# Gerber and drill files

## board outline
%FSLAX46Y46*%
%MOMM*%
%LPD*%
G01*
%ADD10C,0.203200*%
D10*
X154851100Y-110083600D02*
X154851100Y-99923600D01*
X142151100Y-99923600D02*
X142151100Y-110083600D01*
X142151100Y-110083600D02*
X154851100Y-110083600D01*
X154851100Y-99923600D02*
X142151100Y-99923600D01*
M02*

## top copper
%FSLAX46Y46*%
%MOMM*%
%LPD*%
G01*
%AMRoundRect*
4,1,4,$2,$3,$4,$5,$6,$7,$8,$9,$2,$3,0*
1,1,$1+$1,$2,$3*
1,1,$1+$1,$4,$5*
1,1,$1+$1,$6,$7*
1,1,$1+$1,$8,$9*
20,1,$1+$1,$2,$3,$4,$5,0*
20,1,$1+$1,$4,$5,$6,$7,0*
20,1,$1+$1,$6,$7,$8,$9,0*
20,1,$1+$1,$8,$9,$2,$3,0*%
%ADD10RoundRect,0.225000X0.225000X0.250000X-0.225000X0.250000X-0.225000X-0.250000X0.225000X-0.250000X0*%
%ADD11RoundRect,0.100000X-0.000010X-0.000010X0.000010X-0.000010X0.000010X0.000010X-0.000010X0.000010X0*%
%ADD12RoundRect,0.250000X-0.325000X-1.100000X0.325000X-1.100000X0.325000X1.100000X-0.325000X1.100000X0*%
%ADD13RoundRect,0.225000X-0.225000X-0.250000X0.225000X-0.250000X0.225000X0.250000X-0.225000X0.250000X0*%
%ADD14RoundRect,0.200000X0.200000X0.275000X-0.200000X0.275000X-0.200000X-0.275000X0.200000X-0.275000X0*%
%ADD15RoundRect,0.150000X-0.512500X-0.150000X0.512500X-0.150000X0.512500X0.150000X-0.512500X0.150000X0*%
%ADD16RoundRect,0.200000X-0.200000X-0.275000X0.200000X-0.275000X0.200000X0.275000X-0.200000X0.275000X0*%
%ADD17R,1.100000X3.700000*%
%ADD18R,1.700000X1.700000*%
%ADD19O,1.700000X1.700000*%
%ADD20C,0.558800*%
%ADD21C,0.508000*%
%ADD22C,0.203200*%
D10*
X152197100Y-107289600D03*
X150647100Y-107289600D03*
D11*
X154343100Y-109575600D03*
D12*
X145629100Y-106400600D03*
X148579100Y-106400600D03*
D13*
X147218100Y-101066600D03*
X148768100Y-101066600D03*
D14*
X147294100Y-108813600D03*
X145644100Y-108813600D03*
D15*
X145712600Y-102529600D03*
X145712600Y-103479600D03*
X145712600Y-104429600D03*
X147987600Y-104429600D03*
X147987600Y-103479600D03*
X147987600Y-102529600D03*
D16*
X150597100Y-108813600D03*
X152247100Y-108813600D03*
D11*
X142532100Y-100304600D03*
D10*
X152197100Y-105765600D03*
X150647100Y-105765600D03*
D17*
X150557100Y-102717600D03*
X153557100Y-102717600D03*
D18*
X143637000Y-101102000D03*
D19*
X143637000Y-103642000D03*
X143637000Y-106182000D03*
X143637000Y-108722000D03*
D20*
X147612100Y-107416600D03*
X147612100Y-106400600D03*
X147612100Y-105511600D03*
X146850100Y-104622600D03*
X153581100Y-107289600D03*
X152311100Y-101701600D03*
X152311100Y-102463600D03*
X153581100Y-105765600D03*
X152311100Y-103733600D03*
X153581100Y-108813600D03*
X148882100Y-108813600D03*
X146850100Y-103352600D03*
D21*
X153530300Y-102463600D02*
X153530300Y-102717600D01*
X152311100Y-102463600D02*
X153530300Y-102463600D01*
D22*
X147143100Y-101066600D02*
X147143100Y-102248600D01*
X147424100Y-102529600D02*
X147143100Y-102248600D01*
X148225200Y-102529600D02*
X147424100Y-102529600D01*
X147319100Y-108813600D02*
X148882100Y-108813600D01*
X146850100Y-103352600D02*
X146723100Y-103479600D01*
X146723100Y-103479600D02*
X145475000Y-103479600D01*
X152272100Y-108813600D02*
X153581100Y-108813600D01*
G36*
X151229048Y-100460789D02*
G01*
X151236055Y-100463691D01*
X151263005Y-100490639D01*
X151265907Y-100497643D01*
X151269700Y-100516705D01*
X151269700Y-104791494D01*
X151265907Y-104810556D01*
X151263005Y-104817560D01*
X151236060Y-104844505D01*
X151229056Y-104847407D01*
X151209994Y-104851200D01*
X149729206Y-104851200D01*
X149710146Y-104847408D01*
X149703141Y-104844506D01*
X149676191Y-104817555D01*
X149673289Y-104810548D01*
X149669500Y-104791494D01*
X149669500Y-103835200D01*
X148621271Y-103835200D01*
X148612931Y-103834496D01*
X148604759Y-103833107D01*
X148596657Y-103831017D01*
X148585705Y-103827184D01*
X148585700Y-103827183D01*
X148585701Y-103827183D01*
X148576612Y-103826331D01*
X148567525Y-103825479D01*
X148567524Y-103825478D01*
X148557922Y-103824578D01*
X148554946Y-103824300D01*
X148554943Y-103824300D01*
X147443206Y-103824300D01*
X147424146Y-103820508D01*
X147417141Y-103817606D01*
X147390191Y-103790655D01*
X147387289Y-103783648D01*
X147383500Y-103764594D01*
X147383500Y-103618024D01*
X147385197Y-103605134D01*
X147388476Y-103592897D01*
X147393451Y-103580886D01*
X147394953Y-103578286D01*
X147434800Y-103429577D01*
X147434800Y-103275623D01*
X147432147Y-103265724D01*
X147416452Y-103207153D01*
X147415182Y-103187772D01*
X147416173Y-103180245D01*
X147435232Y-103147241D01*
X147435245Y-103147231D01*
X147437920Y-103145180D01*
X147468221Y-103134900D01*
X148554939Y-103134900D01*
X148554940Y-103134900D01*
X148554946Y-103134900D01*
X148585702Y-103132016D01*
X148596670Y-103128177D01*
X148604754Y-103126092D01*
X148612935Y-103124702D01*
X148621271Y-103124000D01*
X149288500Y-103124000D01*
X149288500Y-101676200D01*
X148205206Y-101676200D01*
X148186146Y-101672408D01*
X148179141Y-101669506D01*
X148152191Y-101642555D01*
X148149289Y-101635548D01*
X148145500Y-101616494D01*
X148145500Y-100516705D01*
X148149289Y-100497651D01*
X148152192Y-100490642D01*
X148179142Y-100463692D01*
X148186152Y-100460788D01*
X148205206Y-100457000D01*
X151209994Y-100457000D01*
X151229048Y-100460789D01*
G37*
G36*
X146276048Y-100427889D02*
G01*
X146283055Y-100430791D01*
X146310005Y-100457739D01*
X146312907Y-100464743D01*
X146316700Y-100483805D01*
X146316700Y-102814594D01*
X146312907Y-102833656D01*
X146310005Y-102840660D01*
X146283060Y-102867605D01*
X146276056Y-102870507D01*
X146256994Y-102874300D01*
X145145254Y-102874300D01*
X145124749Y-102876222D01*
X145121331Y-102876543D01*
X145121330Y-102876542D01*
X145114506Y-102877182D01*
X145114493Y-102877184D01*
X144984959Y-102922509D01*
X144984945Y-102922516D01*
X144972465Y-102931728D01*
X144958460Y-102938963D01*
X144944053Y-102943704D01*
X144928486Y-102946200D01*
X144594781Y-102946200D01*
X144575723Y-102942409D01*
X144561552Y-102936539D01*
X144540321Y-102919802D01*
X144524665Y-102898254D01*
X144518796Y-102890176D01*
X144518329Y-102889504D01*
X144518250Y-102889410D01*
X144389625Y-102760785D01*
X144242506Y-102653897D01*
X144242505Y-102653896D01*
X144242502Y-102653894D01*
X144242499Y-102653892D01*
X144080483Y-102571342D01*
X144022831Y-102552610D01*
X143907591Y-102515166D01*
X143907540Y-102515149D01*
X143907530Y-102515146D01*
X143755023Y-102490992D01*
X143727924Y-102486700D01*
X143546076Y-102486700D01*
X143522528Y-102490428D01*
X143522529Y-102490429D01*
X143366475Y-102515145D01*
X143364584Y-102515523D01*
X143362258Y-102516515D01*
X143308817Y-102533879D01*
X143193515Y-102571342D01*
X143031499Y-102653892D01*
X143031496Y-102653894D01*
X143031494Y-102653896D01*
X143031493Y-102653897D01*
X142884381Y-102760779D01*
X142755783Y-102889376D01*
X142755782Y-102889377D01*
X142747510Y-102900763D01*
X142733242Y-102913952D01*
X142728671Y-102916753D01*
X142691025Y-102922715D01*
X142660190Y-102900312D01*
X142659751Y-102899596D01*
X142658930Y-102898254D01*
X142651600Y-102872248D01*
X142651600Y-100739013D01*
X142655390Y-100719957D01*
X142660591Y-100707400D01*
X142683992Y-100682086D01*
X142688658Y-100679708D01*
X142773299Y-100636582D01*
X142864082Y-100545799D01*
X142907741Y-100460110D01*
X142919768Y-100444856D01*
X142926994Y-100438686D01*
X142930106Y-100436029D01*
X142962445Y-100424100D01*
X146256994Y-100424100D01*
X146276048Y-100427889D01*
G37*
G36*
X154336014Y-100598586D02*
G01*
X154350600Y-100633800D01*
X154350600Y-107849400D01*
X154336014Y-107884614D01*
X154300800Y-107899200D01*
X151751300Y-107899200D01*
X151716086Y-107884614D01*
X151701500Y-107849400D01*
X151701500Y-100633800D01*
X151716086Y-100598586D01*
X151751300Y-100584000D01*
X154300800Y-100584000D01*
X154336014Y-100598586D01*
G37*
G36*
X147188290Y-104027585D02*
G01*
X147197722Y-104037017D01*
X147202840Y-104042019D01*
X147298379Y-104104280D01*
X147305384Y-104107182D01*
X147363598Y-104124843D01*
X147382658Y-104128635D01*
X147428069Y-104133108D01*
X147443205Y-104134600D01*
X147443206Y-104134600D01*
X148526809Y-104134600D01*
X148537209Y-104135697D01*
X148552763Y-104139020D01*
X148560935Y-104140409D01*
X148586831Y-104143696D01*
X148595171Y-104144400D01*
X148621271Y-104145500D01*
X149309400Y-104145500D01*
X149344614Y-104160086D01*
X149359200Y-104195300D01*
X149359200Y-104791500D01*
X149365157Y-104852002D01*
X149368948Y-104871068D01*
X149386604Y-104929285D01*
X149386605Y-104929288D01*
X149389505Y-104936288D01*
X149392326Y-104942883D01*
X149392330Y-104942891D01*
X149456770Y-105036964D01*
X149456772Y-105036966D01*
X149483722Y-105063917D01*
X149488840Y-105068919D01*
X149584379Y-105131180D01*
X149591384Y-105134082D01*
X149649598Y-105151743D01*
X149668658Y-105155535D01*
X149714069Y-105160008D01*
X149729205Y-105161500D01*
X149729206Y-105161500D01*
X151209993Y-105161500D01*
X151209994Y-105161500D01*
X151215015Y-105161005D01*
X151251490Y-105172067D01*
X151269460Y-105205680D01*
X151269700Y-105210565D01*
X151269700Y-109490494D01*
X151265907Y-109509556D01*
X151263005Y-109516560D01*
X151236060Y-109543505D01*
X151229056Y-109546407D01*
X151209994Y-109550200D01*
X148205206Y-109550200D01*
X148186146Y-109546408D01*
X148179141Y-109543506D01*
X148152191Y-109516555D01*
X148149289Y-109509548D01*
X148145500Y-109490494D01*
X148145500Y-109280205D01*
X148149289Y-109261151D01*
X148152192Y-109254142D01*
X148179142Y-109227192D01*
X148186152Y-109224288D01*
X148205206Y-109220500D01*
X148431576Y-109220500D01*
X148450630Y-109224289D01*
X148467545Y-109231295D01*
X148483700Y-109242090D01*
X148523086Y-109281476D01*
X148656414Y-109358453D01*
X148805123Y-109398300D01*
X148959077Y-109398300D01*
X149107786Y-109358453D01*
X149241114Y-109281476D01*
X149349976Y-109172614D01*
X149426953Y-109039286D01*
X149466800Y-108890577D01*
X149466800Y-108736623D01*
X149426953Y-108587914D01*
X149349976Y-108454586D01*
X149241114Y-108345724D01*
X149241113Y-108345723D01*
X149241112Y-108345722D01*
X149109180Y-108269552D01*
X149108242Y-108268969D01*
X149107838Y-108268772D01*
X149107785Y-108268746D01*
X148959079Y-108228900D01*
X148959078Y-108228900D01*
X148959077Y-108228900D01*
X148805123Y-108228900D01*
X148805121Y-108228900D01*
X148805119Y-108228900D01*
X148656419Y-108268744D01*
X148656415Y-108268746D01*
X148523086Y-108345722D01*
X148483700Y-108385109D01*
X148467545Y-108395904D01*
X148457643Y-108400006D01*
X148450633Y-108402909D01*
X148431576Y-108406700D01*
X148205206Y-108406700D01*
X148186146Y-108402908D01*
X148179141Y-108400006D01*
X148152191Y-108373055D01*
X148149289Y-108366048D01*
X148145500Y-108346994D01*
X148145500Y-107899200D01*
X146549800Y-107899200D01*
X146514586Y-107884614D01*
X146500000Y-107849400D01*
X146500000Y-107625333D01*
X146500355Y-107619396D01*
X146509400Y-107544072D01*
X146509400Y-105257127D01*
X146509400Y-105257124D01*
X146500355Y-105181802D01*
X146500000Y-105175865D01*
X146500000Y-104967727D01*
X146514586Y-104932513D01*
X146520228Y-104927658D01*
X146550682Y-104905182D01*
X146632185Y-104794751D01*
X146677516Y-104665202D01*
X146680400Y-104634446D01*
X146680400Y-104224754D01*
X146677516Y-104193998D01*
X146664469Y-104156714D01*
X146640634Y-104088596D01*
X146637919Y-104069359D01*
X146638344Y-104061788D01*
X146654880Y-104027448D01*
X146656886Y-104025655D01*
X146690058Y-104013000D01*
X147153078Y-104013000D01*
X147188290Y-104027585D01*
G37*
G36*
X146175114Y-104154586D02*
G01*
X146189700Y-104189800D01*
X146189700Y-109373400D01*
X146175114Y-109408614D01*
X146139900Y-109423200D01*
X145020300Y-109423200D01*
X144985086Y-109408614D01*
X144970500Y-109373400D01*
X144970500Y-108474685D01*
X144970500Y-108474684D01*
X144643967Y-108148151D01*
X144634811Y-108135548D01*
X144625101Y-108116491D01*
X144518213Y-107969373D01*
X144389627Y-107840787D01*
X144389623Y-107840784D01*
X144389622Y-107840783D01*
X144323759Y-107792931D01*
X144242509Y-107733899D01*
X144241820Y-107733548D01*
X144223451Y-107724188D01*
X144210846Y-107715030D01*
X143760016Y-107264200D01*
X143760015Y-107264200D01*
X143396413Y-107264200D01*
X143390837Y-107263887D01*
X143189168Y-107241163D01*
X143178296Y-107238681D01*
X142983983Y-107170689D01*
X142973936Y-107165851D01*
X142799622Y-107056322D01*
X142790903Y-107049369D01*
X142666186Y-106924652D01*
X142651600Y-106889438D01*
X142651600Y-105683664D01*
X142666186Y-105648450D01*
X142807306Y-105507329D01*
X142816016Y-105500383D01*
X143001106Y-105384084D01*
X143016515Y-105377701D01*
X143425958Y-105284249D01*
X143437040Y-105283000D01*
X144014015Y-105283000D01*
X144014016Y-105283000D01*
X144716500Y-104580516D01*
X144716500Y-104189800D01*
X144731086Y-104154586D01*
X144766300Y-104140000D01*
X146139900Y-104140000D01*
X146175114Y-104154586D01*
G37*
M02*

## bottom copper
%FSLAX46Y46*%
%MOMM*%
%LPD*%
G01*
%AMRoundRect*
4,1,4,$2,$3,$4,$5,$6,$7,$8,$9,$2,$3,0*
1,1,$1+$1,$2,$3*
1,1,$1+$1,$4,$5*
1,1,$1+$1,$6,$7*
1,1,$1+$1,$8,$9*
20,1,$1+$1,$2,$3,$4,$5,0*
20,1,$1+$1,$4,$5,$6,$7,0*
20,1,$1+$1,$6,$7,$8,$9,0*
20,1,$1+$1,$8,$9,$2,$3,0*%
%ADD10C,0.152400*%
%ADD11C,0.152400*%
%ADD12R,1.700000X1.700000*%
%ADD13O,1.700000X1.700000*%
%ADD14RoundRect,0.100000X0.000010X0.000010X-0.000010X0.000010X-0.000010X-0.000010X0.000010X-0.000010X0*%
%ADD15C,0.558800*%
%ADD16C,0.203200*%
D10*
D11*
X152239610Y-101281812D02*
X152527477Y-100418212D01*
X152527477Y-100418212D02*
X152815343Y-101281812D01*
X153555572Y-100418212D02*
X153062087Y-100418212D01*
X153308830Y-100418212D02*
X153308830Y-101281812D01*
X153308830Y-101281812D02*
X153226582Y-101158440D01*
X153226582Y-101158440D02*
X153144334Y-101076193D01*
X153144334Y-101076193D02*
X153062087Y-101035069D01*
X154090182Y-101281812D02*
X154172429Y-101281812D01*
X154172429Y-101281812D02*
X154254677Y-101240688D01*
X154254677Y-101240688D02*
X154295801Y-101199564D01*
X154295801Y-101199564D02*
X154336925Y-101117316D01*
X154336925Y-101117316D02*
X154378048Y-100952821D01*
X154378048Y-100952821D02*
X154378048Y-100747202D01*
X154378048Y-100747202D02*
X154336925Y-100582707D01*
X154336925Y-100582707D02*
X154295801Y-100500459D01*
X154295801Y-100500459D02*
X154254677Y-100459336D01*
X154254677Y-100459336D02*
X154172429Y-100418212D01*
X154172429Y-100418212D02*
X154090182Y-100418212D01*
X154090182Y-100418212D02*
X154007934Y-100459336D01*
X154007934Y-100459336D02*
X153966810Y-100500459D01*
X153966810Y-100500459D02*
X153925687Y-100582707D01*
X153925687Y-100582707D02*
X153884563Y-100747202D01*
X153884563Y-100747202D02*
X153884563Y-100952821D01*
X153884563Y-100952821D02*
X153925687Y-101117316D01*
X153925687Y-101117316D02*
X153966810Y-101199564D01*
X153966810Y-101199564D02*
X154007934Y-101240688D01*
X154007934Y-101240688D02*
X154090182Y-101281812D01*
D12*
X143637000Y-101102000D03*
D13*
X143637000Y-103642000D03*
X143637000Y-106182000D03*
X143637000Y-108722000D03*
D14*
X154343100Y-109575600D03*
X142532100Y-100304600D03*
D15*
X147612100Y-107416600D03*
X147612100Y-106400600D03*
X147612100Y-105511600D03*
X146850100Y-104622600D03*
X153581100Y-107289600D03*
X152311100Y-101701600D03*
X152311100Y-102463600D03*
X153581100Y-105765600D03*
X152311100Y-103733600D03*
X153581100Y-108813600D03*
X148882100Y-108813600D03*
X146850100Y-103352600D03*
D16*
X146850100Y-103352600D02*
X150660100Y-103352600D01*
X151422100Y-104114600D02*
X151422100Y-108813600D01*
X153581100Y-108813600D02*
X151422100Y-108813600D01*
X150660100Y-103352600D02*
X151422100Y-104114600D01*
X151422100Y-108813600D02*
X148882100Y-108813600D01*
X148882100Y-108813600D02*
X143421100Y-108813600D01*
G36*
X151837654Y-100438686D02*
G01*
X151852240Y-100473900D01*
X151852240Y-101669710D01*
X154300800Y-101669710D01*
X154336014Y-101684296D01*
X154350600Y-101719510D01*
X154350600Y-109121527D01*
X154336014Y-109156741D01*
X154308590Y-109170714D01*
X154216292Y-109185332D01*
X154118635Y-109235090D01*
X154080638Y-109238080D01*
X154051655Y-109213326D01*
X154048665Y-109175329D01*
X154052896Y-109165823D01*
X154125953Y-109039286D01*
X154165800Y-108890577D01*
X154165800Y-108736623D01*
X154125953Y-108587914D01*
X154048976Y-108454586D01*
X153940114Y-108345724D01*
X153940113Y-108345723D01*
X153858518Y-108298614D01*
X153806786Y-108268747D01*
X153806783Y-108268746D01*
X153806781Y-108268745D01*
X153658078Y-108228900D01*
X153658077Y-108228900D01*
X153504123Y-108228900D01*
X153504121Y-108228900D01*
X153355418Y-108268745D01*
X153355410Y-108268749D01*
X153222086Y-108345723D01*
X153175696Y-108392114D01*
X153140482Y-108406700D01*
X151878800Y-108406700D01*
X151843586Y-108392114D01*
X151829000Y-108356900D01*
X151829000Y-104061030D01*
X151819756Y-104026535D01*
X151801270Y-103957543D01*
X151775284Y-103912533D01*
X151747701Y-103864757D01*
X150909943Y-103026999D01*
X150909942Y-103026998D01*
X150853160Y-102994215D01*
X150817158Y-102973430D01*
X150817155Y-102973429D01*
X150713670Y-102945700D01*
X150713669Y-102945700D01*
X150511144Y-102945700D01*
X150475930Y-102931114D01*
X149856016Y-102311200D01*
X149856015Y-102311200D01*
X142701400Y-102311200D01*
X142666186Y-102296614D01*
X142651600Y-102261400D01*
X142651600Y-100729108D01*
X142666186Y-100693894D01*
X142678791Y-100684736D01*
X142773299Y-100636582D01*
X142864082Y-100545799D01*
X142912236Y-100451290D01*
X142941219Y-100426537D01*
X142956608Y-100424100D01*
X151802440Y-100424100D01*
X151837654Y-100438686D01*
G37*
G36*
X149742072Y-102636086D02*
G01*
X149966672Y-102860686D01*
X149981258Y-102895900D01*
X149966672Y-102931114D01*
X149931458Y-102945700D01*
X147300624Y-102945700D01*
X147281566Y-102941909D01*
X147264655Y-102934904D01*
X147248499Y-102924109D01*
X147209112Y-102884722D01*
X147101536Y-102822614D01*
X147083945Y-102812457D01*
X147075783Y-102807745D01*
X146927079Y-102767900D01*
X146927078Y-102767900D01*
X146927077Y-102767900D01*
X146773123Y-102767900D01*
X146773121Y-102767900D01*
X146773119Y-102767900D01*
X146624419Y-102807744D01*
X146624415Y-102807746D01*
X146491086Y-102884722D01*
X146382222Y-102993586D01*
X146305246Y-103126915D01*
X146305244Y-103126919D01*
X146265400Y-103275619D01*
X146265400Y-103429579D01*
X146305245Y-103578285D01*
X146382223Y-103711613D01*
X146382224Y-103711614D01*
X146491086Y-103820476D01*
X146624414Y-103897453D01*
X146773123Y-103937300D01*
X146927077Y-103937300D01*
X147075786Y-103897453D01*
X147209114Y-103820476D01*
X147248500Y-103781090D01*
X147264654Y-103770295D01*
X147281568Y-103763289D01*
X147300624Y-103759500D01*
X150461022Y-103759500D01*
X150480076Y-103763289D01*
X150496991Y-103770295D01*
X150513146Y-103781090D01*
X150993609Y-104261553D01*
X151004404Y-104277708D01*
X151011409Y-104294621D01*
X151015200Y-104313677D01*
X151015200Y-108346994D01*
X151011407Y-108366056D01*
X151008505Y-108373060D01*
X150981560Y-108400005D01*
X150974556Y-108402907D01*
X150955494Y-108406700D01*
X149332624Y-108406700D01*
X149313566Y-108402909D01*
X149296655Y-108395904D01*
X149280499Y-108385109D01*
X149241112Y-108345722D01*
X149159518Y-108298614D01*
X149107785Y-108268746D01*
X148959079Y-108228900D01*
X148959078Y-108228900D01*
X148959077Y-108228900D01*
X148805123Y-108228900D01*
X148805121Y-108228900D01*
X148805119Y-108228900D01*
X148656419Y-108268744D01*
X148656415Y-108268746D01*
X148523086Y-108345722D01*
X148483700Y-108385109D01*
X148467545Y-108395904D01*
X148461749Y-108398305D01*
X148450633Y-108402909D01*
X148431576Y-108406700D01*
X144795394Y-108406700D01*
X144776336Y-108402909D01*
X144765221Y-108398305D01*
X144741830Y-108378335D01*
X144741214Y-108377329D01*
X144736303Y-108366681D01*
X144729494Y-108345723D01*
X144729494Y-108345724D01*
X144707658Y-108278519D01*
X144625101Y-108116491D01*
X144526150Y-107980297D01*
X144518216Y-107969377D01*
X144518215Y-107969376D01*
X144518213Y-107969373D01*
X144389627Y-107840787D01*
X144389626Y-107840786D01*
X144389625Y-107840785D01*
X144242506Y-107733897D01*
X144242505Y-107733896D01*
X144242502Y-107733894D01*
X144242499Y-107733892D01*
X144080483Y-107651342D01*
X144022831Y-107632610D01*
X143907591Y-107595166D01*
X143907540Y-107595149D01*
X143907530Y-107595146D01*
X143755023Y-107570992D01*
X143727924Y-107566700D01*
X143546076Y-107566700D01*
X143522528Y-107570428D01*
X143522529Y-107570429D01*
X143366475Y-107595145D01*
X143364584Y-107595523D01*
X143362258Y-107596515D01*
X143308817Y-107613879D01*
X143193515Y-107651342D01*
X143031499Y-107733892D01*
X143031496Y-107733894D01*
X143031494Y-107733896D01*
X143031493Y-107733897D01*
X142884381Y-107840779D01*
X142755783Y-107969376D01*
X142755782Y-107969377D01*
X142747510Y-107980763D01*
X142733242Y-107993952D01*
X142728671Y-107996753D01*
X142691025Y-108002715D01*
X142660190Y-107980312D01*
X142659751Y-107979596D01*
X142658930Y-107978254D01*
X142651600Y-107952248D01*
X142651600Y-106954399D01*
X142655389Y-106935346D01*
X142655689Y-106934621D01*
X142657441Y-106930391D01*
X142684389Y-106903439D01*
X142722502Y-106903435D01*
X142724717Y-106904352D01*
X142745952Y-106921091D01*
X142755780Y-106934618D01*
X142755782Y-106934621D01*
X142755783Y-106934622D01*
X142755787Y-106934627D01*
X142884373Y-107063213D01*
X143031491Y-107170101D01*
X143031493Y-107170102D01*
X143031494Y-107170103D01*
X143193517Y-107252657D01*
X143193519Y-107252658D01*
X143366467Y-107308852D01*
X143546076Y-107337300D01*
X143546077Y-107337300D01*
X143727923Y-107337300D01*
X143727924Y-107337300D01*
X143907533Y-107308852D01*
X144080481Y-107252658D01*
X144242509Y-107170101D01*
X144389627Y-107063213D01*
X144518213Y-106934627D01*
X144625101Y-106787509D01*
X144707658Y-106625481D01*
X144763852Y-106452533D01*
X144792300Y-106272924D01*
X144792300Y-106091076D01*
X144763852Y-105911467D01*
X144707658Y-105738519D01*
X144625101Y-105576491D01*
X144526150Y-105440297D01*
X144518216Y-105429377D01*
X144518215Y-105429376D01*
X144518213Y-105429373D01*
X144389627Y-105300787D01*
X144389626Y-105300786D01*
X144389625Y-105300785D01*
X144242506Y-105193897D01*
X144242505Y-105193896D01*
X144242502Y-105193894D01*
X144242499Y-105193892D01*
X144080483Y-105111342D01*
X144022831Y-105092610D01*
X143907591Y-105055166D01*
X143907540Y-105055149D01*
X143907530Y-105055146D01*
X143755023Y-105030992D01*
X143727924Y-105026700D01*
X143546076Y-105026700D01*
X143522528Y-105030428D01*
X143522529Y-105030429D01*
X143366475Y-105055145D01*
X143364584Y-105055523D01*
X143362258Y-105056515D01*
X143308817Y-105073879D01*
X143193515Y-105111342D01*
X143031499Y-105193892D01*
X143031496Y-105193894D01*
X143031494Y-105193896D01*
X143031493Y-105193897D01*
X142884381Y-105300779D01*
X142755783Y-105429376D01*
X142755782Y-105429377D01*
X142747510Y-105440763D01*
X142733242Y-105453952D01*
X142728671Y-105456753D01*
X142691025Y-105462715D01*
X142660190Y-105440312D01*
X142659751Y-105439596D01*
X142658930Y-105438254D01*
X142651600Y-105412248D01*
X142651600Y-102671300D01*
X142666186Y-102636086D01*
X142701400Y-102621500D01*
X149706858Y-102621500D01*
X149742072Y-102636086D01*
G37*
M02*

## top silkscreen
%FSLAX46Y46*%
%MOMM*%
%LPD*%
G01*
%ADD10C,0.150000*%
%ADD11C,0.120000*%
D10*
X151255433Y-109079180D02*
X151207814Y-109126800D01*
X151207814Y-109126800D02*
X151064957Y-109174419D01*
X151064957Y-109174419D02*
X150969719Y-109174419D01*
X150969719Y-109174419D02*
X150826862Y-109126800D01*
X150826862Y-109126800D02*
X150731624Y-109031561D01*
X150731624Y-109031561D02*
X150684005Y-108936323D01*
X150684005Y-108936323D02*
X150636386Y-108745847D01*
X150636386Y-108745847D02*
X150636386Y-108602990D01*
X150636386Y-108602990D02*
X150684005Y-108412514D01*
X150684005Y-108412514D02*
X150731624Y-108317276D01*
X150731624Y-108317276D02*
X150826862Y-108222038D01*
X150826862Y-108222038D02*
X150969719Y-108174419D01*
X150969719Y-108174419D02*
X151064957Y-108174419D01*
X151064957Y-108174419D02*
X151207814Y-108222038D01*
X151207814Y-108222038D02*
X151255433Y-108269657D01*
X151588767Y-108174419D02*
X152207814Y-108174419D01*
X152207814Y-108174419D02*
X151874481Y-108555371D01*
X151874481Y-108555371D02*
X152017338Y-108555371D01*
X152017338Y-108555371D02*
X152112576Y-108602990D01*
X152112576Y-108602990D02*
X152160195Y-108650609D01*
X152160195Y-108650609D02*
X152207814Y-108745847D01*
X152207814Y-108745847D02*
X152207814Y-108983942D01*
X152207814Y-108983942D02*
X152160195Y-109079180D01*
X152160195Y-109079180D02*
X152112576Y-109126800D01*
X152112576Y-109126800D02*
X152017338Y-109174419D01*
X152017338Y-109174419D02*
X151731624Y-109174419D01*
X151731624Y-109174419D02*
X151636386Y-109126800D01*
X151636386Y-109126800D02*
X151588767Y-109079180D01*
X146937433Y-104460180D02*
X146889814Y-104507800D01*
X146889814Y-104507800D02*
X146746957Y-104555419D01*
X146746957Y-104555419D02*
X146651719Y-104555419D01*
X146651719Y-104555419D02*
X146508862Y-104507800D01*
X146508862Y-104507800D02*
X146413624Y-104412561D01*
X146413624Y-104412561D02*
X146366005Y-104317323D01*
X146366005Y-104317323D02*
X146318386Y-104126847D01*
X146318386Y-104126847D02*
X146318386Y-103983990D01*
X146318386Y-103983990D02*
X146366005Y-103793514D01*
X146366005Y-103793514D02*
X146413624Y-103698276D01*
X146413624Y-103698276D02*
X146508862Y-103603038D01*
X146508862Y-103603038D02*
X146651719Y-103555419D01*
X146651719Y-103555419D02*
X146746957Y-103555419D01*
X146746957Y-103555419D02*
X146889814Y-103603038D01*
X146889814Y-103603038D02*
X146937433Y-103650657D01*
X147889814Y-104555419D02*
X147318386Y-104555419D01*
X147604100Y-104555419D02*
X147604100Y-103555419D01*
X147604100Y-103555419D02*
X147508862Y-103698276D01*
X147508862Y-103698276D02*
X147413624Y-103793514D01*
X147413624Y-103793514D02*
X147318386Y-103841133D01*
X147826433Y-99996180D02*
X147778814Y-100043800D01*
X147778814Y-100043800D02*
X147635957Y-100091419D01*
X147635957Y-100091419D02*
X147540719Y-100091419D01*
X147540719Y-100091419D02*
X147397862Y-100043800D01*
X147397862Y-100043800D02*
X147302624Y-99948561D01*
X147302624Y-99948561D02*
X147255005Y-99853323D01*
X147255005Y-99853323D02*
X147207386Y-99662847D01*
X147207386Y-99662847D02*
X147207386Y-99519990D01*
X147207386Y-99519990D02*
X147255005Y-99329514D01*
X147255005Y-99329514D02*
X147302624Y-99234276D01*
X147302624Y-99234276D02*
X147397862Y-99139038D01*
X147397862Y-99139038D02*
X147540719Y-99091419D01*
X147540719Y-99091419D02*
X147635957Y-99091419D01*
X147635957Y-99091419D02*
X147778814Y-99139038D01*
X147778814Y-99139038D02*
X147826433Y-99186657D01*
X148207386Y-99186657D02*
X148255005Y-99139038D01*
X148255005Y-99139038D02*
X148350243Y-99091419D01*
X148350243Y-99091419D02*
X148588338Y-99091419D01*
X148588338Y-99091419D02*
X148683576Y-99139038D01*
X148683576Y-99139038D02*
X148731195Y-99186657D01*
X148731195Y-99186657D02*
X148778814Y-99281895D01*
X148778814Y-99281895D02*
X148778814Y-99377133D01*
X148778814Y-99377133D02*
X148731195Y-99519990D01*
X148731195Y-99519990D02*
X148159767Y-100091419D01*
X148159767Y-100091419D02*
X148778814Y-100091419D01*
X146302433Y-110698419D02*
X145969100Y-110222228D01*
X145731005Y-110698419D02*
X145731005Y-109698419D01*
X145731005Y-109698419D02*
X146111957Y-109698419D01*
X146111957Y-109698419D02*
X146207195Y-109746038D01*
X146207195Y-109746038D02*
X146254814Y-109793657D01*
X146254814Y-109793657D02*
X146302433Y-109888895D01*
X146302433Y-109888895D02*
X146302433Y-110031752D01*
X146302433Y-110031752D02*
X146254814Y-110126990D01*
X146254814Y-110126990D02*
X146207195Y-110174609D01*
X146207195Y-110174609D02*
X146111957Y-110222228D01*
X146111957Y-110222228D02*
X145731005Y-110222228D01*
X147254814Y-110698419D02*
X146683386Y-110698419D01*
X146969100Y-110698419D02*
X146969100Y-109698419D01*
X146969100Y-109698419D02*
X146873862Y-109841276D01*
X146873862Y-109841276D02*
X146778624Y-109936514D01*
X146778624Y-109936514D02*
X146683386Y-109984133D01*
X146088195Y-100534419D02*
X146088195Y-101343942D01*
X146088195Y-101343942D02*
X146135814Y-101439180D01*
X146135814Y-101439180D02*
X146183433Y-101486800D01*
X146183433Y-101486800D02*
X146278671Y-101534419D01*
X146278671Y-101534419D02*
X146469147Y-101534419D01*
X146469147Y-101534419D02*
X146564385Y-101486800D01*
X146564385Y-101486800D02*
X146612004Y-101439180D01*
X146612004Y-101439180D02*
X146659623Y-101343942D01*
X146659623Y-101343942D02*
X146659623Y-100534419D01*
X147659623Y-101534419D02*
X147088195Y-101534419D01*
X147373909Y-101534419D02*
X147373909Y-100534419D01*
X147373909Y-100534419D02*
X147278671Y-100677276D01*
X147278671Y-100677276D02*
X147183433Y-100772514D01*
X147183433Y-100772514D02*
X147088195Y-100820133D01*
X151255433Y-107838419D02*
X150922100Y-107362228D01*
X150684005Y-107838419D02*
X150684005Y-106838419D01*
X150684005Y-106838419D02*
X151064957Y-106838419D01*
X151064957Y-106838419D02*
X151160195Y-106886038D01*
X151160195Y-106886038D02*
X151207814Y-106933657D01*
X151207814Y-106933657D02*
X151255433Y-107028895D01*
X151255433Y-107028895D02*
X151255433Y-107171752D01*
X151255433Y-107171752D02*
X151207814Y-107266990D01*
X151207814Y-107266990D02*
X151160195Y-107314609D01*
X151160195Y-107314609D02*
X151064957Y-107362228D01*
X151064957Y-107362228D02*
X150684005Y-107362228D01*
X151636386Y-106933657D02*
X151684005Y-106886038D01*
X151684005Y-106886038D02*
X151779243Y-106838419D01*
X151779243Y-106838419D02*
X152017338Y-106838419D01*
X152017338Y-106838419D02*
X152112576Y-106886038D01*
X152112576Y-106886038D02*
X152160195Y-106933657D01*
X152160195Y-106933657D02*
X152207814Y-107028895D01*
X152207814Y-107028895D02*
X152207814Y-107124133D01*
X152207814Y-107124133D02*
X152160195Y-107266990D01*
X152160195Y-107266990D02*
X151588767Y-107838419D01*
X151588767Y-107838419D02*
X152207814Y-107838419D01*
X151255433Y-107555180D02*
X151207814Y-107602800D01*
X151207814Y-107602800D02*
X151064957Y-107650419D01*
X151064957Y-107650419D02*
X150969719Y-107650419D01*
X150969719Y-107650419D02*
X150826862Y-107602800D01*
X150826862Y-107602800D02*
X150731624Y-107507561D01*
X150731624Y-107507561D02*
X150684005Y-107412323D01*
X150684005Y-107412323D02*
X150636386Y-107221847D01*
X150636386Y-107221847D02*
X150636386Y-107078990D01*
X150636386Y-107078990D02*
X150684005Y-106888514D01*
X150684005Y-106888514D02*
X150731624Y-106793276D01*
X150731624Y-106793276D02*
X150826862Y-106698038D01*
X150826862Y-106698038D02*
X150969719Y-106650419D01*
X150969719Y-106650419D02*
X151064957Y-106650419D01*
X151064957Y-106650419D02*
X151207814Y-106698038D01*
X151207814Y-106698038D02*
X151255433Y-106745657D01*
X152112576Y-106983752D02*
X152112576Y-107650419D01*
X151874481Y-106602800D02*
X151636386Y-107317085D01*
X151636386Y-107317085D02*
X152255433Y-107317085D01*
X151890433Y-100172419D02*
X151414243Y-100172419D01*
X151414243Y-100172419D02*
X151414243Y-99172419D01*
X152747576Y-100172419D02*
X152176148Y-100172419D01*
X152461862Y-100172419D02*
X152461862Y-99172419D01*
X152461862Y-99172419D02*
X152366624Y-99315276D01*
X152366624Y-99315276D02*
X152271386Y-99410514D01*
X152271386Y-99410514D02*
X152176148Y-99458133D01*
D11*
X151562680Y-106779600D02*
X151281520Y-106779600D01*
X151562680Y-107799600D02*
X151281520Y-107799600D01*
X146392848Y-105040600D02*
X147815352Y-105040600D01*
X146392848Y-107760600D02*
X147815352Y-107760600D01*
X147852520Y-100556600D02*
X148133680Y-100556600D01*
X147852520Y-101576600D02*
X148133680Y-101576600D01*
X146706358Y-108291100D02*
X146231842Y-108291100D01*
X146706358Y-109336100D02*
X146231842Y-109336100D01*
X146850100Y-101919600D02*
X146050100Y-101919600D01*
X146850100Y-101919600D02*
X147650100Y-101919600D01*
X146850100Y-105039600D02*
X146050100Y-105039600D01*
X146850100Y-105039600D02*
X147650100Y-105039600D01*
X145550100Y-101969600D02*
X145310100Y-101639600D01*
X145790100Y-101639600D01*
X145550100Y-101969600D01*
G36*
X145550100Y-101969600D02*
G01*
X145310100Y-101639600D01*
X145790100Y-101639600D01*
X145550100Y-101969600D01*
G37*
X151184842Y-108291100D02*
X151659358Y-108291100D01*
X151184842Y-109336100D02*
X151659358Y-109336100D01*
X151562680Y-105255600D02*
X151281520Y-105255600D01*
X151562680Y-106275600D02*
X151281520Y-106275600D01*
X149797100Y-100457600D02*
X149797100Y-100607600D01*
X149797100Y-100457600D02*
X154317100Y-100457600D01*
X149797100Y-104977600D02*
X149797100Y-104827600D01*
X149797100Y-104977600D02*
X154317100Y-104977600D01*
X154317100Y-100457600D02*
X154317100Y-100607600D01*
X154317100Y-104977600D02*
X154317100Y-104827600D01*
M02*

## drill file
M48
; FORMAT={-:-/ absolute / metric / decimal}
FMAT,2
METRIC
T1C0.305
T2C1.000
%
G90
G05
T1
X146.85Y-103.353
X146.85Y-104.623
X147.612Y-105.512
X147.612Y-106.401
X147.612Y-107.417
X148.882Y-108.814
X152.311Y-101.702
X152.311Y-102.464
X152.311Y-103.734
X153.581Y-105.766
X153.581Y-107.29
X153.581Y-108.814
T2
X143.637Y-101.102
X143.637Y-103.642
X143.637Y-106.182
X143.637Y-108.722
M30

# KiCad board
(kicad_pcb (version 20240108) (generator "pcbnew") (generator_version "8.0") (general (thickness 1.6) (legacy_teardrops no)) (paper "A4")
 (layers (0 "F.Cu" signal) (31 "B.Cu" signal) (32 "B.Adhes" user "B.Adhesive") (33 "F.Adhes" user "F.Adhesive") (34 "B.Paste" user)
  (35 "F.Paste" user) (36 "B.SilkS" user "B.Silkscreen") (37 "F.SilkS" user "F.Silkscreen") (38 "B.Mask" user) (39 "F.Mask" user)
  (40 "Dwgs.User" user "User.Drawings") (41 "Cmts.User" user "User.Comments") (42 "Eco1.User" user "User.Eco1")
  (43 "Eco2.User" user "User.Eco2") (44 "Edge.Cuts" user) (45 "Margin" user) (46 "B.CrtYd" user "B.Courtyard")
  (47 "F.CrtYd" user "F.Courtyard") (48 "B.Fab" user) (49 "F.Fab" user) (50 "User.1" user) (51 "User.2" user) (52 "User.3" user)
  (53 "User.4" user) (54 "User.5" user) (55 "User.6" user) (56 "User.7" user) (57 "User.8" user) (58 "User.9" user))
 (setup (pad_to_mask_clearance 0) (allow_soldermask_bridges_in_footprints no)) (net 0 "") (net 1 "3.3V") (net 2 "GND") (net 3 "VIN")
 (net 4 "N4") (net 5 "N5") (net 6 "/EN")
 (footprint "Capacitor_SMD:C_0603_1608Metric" (layer "F.Cu") (at 151.4221 107.2896 180)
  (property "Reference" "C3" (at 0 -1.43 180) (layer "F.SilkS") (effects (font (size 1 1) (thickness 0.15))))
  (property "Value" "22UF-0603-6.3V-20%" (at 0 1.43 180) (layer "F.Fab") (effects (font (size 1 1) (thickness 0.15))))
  (fp_line (start -0.14058 0.51) (end 0.14058 0.51) (stroke (width 0.12) (type solid)) (layer "F.SilkS"))
  (fp_line (start -0.14058 -0.51) (end 0.14058 -0.51) (stroke (width 0.12) (type solid)) (layer "F.SilkS"))
  (pad "1" smd roundrect (at -0.775 0 180) (size 0.9 0.95) (layers "F.Cu" "F.Paste" "F.Mask") (roundrect_rratio 0.25) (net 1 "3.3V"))
  (pad "2" smd roundrect (at 0.775 0 180) (size 0.9 0.95) (layers "F.Cu" "F.Paste" "F.Mask") (roundrect_rratio 0.25) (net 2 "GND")))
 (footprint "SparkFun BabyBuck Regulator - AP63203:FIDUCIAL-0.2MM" (layer "F.Cu") (at 154.3431 109.5756)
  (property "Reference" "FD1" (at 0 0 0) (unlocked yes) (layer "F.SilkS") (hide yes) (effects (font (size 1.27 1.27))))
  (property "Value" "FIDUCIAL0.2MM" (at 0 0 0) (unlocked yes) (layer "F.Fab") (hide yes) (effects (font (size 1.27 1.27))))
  (pad "1" smd roundrect (at 0 0) (size 0.2 0.2) (layers "F.Cu") (roundrect_rratio 0.5) (solder_mask_margin 0.0635) (thermal_bridge_angle 0)))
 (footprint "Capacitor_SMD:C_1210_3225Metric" (layer "F.Cu") (at 147.1041 106.4006)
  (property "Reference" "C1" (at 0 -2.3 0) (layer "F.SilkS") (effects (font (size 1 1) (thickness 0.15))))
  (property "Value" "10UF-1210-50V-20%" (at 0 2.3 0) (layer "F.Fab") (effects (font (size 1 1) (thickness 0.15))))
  (fp_line (start -0.711252 -1.36) (end 0.711252 -1.36) (stroke (width 0.12) (type solid)) (layer "F.SilkS"))
  (fp_line (start -0.711252 1.36) (end 0.711252 1.36) (stroke (width 0.12) (type solid)) (layer "F.SilkS"))
  (pad "1" smd roundrect (at -1.475 0) (size 1.15 2.7) (layers "F.Cu" "F.Paste" "F.Mask") (roundrect_rratio 0.217391) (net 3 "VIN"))
  (pad "2" smd roundrect (at 1.475 0) (size 1.15 2.7) (layers "F.Cu" "F.Paste" "F.Mask") (roundrect_rratio 0.217391) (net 2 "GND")))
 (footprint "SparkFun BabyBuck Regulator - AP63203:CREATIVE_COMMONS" (layer "F.Cu") (at 125.6411 125.3236)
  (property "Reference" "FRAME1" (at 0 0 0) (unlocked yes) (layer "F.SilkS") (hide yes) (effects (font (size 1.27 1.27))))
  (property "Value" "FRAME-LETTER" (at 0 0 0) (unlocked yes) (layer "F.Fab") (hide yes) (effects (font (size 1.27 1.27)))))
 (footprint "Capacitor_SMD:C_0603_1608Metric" (layer "F.Cu") (at 147.9931 101.0666)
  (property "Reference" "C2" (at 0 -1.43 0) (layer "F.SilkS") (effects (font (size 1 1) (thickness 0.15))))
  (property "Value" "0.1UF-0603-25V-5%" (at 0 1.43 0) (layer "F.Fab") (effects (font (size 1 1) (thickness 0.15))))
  (fp_line (start -0.14058 -0.51) (end 0.14058 -0.51) (stroke (width 0.12) (type solid)) (layer "F.SilkS"))
  (fp_line (start -0.14058 0.51) (end 0.14058 0.51) (stroke (width 0.12) (type solid)) (layer "F.SilkS"))
  (pad "1" smd roundrect (at -0.775 0) (size 0.9 0.95) (layers "F.Cu" "F.Paste" "F.Mask") (roundrect_rratio 0.25) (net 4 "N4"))
  (pad "2" smd roundrect (at 0.775 0) (size 0.9 0.95) (layers "F.Cu" "F.Paste" "F.Mask") (roundrect_rratio 0.25) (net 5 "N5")))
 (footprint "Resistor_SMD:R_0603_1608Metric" (layer "F.Cu") (at 146.4691 108.8136 180)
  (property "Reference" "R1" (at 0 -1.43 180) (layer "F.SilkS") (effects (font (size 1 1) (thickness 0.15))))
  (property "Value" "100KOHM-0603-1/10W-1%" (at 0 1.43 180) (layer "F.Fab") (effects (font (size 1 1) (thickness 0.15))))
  (fp_line (start -0.237258 0.5225) (end 0.237258 0.5225) (stroke (width 0.12) (type solid)) (layer "F.SilkS"))
  (fp_line (start -0.237258 -0.5225) (end 0.237258 -0.5225) (stroke (width 0.12) (type solid)) (layer "F.SilkS"))
  (pad "1" smd roundrect (at -0.825 0 180) (size 0.8 0.95) (layers "F.Cu" "F.Paste" "F.Mask") (roundrect_rratio 0.25) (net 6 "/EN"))
  (pad "2" smd roundrect (at 0.825 0 180) (size 0.8 0.95) (layers "F.Cu" "F.Paste" "F.Mask") (roundrect_rratio 0.25) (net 3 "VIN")))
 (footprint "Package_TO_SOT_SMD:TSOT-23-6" (layer "F.Cu") (at 146.8501 103.4796)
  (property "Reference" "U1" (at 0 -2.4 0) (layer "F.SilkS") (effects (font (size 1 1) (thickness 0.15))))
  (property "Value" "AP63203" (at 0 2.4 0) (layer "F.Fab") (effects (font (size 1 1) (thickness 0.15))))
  (fp_line (start 0 -1.56) (end -0.8 -1.56) (stroke (width 0.12) (type solid)) (layer "F.SilkS"))
  (fp_line (start 0 -1.56) (end 0.8 -1.56) (stroke (width 0.12) (type solid)) (layer "F.SilkS"))
  (fp_line (start 0 1.56) (end -0.8 1.56) (stroke (width 0.12) (type solid)) (layer "F.SilkS"))
  (fp_line (start 0 1.56) (end 0.8 1.56) (stroke (width 0.12) (type solid)) (layer "F.SilkS"))
  (fp_poly
   (pts (xy -1.3 -1.51) (xy -1.54 -1.84) (xy -1.06 -1.84) (xy -1.3 -1.51)) (stroke (width 0.12) (type solid)) (fill solid) (layer "F.SilkS"))
  (pad "1" smd roundrect (at -1.1375 -0.95) (size 1.325 0.6) (layers "F.Cu" "F.Paste" "F.Mask") (roundrect_rratio 0.25) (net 1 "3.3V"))
  (pad "2" smd roundrect (at -1.1375 0) (size 1.325 0.6) (layers "F.Cu" "F.Paste" "F.Mask") (roundrect_rratio 0.25) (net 6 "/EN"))
  (pad "3" smd roundrect (at -1.1375 0.95) (size 1.325 0.6) (layers "F.Cu" "F.Paste" "F.Mask") (roundrect_rratio 0.25) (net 3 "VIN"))
  (pad "4" smd roundrect (at 1.1375 0.95) (size 1.325 0.6) (layers "F.Cu" "F.Paste" "F.Mask") (roundrect_rratio 0.25) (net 2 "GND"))
  (pad "5" smd roundrect (at 1.1375 0) (size 1.325 0.6) (layers "F.Cu" "F.Paste" "F.Mask") (roundrect_rratio 0.25) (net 5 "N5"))
  (pad "6" smd roundrect (at 1.1375 -0.95) (size 1.325 0.6) (layers "F.Cu" "F.Paste" "F.Mask") (roundrect_rratio 0.25) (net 4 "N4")))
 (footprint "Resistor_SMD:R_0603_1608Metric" (layer "F.Cu") (at 151.4221 108.8136)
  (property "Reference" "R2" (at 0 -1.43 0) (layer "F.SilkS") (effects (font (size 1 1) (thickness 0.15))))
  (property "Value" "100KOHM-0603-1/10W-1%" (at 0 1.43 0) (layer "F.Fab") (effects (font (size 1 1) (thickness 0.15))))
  (fp_line (start -0.237258 -0.5225) (end 0.237258 -0.5225) (stroke (width 0.12) (type solid)) (layer "F.SilkS"))
  (fp_line (start -0.237258 0.5225) (end 0.237258 0.5225) (stroke (width 0.12) (type solid)) (layer "F.SilkS"))
  (pad "1" smd roundrect (at -0.825 0) (size 0.8 0.95) (layers "F.Cu" "F.Paste" "F.Mask") (roundrect_rratio 0.25) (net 2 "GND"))
  (pad "2" smd roundrect (at 0.825 0) (size 0.8 0.95) (layers "F.Cu" "F.Paste" "F.Mask") (roundrect_rratio 0.25) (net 6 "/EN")))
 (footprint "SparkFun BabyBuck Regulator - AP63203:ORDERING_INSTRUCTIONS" (layer "F.Cu") (at 166.2811 65.6336)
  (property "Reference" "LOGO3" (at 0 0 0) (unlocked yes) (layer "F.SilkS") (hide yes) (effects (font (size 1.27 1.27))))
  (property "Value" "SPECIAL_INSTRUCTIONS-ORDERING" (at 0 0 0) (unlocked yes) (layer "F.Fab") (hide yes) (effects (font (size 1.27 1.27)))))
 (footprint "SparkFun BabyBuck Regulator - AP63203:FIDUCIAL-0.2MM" (layer "F.Cu") (at 142.5321 100.3046)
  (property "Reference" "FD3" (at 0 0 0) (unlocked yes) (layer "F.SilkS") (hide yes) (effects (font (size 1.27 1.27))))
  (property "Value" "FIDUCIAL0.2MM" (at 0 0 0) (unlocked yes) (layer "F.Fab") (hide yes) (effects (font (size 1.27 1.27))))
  (pad "1" smd roundrect (at 0 0) (size 0.2 0.2) (layers "F.Cu") (roundrect_rratio 0.5) (solder_mask_margin 0.0635) (thermal_bridge_angle 0)))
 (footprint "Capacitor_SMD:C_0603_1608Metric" (layer "F.Cu") (at 151.4221 105.7656 180)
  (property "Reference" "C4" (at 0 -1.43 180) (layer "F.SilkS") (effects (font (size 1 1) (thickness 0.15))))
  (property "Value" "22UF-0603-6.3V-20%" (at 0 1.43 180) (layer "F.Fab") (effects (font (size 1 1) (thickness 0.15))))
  (fp_line (start -0.14058 0.51) (end 0.14058 0.51) (stroke (width 0.12) (type solid)) (layer "F.SilkS"))
  (fp_line (start -0.14058 -0.51) (end 0.14058 -0.51) (stroke (width 0.12) (type solid)) (layer "F.SilkS"))
  (pad "1" smd roundrect (at -0.775 0 180) (size 0.9 0.95) (layers "F.Cu" "F.Paste" "F.Mask") (roundrect_rratio 0.25) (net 1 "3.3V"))
  (pad "2" smd roundrect (at 0.775 0 180) (size 0.9 0.95) (layers "F.Cu" "F.Paste" "F.Mask") (roundrect_rratio 0.25) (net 2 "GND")))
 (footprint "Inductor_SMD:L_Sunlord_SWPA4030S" (layer "F.Cu") (at 152.0571 102.7176)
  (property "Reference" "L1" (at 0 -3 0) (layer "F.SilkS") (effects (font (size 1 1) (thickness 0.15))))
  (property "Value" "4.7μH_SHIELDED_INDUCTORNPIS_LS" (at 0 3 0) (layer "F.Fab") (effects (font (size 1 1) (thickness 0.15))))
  (fp_line (start -2.26 -2.26) (end -2.26 -2.11) (stroke (width 0.12) (type solid)) (layer "F.SilkS"))
  (fp_line (start -2.26 -2.26) (end 2.26 -2.26) (stroke (width 0.12) (type solid)) (layer "F.SilkS"))
  (fp_line (start -2.26 2.26) (end -2.26 2.11) (stroke (width 0.12) (type solid)) (layer "F.SilkS"))
  (fp_line (start -2.26 2.26) (end 2.26 2.26) (stroke (width 0.12) (type solid)) (layer "F.SilkS"))
  (fp_line (start 2.26 -2.26) (end 2.26 -2.11) (stroke (width 0.12) (type solid)) (layer "F.SilkS"))
  (fp_line (start 2.26 2.26) (end 2.26 2.11) (stroke (width 0.12) (type solid)) (layer "F.SilkS"))
  (pad "1" smd rect (at -1.5 0) (size 1.1 3.7) (layers "F.Cu" "F.Paste" "F.Mask") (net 5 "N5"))
  (pad "2" smd rect (at 1.5 0) (size 1.1 3.7) (layers "F.Cu" "F.Paste" "F.Mask") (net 1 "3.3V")))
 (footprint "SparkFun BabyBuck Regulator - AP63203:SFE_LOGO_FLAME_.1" (layer "B.Cu") (at 149.8981 107.0356 180)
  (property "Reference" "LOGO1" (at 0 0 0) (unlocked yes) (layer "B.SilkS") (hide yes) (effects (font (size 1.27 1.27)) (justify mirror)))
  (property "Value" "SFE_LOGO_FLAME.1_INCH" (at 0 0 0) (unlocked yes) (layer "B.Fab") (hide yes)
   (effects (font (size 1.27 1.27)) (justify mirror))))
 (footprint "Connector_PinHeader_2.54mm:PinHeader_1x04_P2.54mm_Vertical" (layer "B.Cu") (at 143.637 101.102 180)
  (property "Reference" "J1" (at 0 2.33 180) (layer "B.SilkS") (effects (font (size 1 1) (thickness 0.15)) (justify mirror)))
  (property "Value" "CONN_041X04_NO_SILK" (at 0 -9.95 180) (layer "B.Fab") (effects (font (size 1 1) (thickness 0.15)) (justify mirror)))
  (pad "1" thru_hole rect (at 0 0 180) (size 1.7 1.7) (drill 1) (layers "*.Cu" "*.Mask") (remove_unused_layers no) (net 1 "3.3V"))
  (pad "2" thru_hole oval (at 0 -2.54 180) (size 1.7 1.7) (drill 1) (layers "*.Cu" "*.Mask") (remove_unused_layers no) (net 2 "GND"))
  (pad "3" thru_hole oval (at 0 -5.08 180) (size 1.7 1.7) (drill 1) (layers "*.Cu" "*.Mask") (remove_unused_layers no) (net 3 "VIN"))
  (pad "4" thru_hole oval (at 0 -7.62 180) (size 1.7 1.7) (drill 1) (layers "*.Cu" "*.Mask") (remove_unused_layers no) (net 6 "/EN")))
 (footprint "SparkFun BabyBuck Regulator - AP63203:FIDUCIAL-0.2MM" (layer "B.Cu") (at 154.3431 109.5756 180)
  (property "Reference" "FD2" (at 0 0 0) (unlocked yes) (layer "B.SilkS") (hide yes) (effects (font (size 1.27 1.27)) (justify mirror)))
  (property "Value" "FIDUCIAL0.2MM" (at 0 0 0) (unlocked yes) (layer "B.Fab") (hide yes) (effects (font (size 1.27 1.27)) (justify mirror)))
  (pad "1" smd roundrect (at 0 0 180) (size 0.2 0.2) (layers "B.Cu") (roundrect_rratio 0.5) (solder_mask_margin 0.0635)
   (thermal_bridge_angle 0)))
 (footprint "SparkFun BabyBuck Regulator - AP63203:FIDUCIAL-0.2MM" (layer "B.Cu") (at 142.5321 100.3046 180)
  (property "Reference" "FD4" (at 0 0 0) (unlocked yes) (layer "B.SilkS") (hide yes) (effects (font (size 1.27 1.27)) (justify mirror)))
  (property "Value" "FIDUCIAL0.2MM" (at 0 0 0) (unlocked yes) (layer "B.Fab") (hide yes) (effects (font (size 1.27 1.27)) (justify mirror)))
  (pad "1" smd roundrect (at 0 0 180) (size 0.2 0.2) (layers "B.Cu") (roundrect_rratio 0.5) (solder_mask_margin 0.0635)
   (thermal_bridge_angle 0)))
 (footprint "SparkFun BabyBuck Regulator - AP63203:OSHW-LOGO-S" (layer "B.Cu") (at 152.8191 107.0356 180)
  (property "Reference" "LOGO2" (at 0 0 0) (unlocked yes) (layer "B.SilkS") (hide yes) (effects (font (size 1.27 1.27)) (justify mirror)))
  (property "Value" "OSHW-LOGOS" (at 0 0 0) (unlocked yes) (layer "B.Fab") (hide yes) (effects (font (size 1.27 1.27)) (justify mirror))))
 (gr_line (start 154.8511 110.0836) (end 154.8511 99.9236) (stroke (width 0.2032) (type solid)) (layer "Edge.Cuts"))
 (gr_line (start 142.1511 99.9236) (end 142.1511 110.0836) (stroke (width 0.2032) (type solid)) (layer "Edge.Cuts"))
 (gr_line (start 142.1511 110.0836) (end 154.8511 110.0836) (stroke (width 0.2032) (type solid)) (layer "Edge.Cuts"))
 (gr_line (start 154.8511 99.9236) (end 142.1511 99.9236) (stroke (width 0.2032) (type solid)) (layer "Edge.Cuts"))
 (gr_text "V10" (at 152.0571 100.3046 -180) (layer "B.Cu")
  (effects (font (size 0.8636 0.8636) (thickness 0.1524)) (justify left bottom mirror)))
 (via (at 147.6121 107.4166) (size 0.5588) (drill 0.3048) (layers "F.Cu" "B.Cu") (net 2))
 (via (at 147.6121 106.4006) (size 0.5588) (drill 0.3048) (layers "F.Cu" "B.Cu") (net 2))
 (via (at 147.6121 105.5116) (size 0.5588) (drill 0.3048) (layers "F.Cu" "B.Cu") (free yes) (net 2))
 (via (at 146.8501 104.6226) (size 0.5588) (drill 0.3048) (layers "F.Cu" "B.Cu") (free yes) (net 2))
 (segment (start 153.5303 102.4636) (end 153.5303 102.7176) (width 0.508) (layer "F.Cu") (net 1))
 (segment (start 152.3111 102.4636) (end 153.5303 102.4636) (width 0.508) (layer "F.Cu") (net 1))
 (via (at 153.5811 107.2896) (size 0.5588) (drill 0.3048) (layers "F.Cu" "B.Cu") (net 1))
 (via (at 152.3111 101.7016) (size 0.5588) (drill 0.3048) (layers "F.Cu" "B.Cu") (free yes) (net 1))
 (via (at 152.3111 102.4636) (size 0.5588) (drill 0.3048) (layers "F.Cu" "B.Cu") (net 1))
 (via (at 153.5811 105.7656) (size 0.5588) (drill 0.3048) (layers "F.Cu" "B.Cu") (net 1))
 (via (at 152.3111 103.7336) (size 0.5588) (drill 0.3048) (layers "F.Cu" "B.Cu") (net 1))
 (segment (start 147.1431 101.0666) (end 147.1431 102.2486) (width 0.2032) (layer "F.Cu") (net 4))
 (segment (start 147.4241 102.5296) (end 147.1431 102.2486) (width 0.2032) (layer "F.Cu") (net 4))
 (segment (start 148.2252 102.5296) (end 147.4241 102.5296) (width 0.2032) (layer "F.Cu") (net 4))
 (segment (start 147.3191 108.8136) (end 148.8821 108.8136) (width 0.2032) (layer "F.Cu") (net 6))
 (segment (start 146.8501 103.3526) (end 146.7231 103.4796) (width 0.2032) (layer "F.Cu") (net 6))
 (segment (start 146.7231 103.4796) (end 145.475 103.4796) (width 0.2032) (layer "F.Cu") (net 6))
 (segment (start 152.2721 108.8136) (end 153.5811 108.8136) (width 0.2032) (layer "F.Cu") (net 6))
 (via (at 153.5811 108.8136) (size 0.5588) (drill 0.3048) (layers "F.Cu" "B.Cu") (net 6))
 (via (at 148.8821 108.8136) (size 0.5588) (drill 0.3048) (layers "F.Cu" "B.Cu") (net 6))
 (via (at 146.8501 103.3526) (size 0.5588) (drill 0.3048) (layers "F.Cu" "B.Cu") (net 6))
 (segment (start 146.8501 103.3526) (end 150.6601 103.3526) (width 0.2032) (layer "B.Cu") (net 6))
 (segment (start 151.4221 104.1146) (end 151.4221 108.8136) (width 0.2032) (layer "B.Cu") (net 6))
 (segment (start 153.5811 108.8136) (end 151.4221 108.8136) (width 0.2032) (layer "B.Cu") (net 6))
 (segment (start 150.6601 103.3526) (end 151.4221 104.1146) (width 0.2032) (layer "B.Cu") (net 6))
 (segment (start 151.4221 108.8136) (end 148.8821 108.8136) (width 0.2032) (layer "B.Cu") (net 6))
 (segment (start 148.8821 108.8136) (end 143.4211 108.8136) (width 0.2032) (layer "B.Cu") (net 6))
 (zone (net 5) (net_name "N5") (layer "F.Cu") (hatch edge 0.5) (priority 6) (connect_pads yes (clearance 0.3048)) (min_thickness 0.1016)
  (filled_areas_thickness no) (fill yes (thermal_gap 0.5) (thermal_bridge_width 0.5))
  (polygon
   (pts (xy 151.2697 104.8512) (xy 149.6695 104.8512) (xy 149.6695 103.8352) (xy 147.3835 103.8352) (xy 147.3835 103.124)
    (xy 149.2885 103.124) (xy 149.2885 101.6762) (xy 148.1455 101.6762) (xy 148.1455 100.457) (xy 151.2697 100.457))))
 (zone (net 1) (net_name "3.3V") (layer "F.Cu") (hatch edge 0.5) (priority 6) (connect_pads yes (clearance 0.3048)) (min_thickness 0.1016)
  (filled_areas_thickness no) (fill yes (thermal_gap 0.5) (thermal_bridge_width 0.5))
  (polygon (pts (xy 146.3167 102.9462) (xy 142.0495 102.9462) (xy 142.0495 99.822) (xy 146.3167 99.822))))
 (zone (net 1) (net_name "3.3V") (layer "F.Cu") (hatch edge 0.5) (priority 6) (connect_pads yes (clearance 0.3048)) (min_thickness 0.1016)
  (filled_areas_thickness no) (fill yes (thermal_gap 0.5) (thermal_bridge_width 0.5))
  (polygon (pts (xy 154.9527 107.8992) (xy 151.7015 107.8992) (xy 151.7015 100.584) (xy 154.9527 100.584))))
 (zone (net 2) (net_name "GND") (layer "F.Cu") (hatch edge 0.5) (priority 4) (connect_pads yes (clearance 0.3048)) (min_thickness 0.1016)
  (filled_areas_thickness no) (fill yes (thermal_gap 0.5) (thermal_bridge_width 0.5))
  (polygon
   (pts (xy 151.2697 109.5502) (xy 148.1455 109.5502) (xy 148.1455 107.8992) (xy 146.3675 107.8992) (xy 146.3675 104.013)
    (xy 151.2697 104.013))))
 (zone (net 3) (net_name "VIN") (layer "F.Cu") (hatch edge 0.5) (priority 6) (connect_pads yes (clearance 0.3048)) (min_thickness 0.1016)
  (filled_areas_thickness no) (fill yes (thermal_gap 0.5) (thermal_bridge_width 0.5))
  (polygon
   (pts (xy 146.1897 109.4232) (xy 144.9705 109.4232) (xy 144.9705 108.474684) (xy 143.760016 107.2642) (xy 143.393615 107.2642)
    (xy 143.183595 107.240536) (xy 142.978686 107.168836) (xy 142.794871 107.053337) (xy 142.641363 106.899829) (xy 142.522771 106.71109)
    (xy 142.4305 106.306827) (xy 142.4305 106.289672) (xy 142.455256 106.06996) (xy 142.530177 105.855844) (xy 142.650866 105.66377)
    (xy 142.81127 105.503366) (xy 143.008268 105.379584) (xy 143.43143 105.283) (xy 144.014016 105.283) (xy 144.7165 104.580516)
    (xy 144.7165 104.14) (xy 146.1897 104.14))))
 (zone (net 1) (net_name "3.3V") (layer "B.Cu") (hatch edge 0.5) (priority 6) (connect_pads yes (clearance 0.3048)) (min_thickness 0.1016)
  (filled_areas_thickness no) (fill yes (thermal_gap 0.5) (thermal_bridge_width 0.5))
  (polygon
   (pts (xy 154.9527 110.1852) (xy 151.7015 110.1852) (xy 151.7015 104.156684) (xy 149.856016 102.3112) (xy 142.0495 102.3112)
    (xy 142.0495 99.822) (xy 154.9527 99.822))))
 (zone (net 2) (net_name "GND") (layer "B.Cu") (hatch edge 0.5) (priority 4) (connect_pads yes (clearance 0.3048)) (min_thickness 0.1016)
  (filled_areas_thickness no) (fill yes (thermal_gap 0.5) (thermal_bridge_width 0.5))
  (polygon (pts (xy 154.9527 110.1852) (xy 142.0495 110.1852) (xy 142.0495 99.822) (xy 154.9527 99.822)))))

